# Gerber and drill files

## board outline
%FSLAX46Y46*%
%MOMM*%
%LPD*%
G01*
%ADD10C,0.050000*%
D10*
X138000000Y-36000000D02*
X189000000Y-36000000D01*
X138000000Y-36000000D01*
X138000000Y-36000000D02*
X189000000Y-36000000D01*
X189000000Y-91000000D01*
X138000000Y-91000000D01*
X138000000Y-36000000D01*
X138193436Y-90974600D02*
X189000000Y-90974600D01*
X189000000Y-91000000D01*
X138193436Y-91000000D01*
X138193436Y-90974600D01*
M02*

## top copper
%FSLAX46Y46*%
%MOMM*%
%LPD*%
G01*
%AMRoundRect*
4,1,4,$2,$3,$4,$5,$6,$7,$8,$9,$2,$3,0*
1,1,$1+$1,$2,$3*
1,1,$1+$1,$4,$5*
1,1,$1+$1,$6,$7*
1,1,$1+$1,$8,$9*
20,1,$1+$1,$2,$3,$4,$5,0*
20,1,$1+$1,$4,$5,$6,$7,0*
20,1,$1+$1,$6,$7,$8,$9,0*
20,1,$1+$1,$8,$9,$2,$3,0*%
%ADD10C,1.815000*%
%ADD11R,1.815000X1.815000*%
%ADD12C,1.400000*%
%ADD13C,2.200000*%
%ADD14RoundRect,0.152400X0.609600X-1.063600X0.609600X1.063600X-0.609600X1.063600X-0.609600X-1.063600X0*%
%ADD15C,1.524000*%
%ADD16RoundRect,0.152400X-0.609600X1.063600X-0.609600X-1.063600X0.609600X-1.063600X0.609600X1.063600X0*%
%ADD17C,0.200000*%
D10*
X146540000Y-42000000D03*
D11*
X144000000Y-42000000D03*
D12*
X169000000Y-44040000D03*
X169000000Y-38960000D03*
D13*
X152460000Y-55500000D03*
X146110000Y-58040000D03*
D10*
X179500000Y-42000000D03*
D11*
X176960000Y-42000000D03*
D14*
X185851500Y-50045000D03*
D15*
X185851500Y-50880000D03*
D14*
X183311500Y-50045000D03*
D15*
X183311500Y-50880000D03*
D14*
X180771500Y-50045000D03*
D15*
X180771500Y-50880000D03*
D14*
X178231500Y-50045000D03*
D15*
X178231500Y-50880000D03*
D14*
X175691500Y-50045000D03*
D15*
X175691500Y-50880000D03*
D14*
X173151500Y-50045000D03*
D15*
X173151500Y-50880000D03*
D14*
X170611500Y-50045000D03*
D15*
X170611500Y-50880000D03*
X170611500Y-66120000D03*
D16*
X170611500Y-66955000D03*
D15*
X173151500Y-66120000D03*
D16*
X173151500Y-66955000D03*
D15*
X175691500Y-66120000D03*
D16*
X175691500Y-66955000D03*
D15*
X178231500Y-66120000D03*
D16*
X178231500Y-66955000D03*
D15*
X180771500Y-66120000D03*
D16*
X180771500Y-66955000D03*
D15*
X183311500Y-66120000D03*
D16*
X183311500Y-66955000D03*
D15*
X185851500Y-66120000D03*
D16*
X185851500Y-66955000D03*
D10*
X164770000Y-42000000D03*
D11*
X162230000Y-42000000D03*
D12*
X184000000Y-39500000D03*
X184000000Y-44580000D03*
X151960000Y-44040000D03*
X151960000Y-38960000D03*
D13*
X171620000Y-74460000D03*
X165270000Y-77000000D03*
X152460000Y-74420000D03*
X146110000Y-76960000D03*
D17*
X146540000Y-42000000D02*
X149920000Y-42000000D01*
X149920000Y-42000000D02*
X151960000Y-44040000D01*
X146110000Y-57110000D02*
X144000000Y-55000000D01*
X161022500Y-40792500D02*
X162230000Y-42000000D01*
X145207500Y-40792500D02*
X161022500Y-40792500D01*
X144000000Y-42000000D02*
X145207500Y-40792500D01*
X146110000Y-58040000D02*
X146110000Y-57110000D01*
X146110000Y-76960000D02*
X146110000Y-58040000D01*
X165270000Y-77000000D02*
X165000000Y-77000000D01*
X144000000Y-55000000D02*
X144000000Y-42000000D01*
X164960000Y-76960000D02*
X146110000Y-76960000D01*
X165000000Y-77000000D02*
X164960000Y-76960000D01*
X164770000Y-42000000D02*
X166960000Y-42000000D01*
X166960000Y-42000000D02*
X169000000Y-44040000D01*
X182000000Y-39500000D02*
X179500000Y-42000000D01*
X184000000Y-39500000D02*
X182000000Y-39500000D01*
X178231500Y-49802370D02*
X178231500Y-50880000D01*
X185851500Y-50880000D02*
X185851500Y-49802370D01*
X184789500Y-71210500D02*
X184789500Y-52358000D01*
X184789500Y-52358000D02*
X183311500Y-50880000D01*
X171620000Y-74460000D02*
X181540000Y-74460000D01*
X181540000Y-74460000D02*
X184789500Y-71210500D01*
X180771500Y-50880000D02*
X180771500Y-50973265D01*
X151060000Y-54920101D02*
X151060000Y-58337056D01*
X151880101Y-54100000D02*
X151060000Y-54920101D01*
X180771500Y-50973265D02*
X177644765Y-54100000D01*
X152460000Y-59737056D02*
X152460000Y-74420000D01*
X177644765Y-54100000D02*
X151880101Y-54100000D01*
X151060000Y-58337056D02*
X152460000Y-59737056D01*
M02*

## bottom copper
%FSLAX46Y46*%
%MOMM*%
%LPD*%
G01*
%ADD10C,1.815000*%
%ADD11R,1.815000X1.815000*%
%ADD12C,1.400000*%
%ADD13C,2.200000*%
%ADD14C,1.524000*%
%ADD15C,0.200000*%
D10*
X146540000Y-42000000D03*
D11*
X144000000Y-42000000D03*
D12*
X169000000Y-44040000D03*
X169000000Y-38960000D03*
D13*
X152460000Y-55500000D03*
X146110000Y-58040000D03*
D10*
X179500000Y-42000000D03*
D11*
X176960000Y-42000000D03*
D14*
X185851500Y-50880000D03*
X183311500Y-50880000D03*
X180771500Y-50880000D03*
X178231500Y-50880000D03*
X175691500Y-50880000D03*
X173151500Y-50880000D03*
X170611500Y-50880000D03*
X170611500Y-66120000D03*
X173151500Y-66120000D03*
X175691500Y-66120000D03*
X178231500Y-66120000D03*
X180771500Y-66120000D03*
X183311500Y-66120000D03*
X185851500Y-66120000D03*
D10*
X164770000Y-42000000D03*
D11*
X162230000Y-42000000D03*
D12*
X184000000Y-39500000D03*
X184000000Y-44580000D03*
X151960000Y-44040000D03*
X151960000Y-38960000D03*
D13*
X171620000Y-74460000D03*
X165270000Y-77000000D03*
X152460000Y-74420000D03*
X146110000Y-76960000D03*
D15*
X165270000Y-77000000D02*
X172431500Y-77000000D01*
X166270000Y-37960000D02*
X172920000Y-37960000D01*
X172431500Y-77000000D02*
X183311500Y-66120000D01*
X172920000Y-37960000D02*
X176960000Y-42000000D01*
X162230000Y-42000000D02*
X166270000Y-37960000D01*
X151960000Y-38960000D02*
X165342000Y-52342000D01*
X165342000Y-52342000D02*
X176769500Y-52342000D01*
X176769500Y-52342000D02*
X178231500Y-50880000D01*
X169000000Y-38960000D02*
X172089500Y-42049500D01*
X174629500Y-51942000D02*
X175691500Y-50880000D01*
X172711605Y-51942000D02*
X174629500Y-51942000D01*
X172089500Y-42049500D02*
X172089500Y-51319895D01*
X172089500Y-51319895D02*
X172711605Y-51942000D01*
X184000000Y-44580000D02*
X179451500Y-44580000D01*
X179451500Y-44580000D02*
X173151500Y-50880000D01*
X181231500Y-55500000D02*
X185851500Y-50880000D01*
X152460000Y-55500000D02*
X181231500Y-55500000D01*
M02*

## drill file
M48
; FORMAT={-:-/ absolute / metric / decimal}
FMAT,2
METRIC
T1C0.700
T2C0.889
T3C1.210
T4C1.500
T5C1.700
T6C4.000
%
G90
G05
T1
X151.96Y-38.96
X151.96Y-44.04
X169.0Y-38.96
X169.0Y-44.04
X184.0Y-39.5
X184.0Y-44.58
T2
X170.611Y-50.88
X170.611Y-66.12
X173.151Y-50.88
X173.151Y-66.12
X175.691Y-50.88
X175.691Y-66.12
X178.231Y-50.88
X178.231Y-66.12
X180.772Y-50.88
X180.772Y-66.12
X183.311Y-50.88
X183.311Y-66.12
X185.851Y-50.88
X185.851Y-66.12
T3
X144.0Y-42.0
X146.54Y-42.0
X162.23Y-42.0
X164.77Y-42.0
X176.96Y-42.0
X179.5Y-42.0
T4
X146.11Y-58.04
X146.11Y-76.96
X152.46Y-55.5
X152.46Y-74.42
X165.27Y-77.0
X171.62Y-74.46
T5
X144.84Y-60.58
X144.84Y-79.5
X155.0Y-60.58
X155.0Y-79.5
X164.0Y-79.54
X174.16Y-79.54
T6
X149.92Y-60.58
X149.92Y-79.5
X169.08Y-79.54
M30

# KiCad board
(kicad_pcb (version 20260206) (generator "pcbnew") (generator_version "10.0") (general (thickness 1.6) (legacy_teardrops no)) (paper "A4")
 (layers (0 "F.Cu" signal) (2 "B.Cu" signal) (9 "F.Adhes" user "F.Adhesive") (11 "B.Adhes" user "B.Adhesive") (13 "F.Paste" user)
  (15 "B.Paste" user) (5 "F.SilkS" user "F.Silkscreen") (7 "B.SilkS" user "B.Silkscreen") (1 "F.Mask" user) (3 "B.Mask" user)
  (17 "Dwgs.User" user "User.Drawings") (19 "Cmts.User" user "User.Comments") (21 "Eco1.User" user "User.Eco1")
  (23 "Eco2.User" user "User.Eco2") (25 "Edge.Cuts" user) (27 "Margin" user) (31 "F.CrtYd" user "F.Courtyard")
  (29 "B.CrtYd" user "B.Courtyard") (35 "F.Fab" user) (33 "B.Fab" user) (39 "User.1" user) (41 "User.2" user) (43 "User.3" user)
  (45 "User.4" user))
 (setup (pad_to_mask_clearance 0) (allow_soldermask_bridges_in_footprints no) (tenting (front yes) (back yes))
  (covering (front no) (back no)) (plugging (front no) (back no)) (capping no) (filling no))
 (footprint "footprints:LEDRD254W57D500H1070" (layer "F.Cu") (at 145.27 42)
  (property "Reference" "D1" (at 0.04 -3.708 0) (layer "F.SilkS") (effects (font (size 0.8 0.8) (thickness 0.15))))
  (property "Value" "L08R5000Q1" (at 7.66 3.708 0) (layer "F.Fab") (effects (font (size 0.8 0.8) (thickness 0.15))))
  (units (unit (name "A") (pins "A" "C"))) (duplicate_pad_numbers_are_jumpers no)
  (pad "A" thru_hole circle (at 1.27 0) (size 1.815 1.815) (drill 1.21) (layers "*.Cu" "*.Mask") (remove_unused_layers no)
   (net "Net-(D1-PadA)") (solder_mask_margin 0.102))
  (pad "C" thru_hole rect (at -1.27 0) (size 1.815 1.815) (drill 1.21) (layers "*.Cu" "*.Mask") (remove_unused_layers no) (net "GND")
   (solder_mask_margin 0.102)))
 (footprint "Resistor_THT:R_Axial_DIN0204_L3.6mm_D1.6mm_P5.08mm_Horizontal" (layer "F.Cu") (at 169 44.04 90)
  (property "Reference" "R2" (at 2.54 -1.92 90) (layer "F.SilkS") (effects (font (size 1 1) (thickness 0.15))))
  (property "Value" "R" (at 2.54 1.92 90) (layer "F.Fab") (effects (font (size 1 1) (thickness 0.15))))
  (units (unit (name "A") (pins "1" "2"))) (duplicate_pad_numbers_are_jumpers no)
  (pad "1" thru_hole circle (at 0 0 90) (size 1.4 1.4) (drill 0.7) (layers "*.Cu" "*.Mask") (remove_unused_layers no) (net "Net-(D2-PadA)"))
  (pad "2" thru_hole circle (at 5.08 0 90) (size 1.4 1.4) (drill 0.7) (layers "*.Cu" "*.Mask") (remove_unused_layers no) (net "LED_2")))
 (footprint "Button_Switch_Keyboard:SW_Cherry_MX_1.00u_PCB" (layer "F.Cu") (at 152.46 55.5)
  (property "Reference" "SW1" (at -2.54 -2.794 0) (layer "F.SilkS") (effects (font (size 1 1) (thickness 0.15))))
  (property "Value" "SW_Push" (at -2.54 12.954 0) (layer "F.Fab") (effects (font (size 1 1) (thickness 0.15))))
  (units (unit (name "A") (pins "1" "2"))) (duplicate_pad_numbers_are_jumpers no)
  (pad "" np_thru_hole circle (at -7.62 5.08) (size 1.7 1.7) (drill 1.7) (layers "*.Cu" "*.Mask"))
  (pad "" np_thru_hole circle (at -2.54 5.08) (size 4 4) (drill 4) (layers "*.Cu" "*.Mask"))
  (pad "" np_thru_hole circle (at 2.54 5.08) (size 1.7 1.7) (drill 1.7) (layers "*.Cu" "*.Mask"))
  (pad "1" thru_hole circle (at 0 0) (size 2.2 2.2) (drill 1.5) (layers "*.Cu" "*.Mask") (remove_unused_layers no) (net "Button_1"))
  (pad "2" thru_hole circle (at -6.35 2.54) (size 2.2 2.2) (drill 1.5) (layers "*.Cu" "*.Mask") (remove_unused_layers no) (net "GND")))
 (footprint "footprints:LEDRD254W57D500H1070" (layer "F.Cu") (at 178.23 42)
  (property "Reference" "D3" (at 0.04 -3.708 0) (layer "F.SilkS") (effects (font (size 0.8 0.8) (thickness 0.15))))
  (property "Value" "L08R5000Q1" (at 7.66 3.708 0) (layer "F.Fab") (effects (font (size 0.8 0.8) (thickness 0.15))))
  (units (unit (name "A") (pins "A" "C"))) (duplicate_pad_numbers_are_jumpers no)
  (pad "A" thru_hole circle (at 1.27 0) (size 1.815 1.815) (drill 1.21) (layers "*.Cu" "*.Mask") (remove_unused_layers no)
   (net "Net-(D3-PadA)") (solder_mask_margin 0.102))
  (pad "C" thru_hole rect (at -1.27 0) (size 1.815 1.815) (drill 1.21) (layers "*.Cu" "*.Mask") (remove_unused_layers no) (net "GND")
   (solder_mask_margin 0.102)))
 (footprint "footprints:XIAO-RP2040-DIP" (layer "F.Cu") (at 178.2315 58.5)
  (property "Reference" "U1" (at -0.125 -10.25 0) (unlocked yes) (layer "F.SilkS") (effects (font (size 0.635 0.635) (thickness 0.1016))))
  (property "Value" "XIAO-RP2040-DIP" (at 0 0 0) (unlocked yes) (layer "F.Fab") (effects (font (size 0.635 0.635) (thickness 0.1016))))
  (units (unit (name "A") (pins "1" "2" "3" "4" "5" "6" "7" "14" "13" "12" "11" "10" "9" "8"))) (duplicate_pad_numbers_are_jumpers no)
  (pad "1" smd roundrect (at 7.62 -8.455 90) (size 2.432 1.524) (layers "F.Cu" "F.Mask") (roundrect_rratio 0.1) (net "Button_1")
   (thermal_bridge_angle 45))
  (pad "1" thru_hole circle (at 7.62 -7.62 90) (size 1.524 1.524) (drill 0.889) (layers "*.Cu" "*.Mask") (remove_unused_layers no)
   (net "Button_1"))
  (pad "2" smd roundrect (at 5.08 -8.455 90) (size 2.432 1.524) (layers "F.Cu" "F.Mask") (roundrect_rratio 0.1) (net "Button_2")
   (thermal_bridge_angle 45))
  (pad "2" thru_hole circle (at 5.08 -7.62 90) (size 1.524 1.524) (drill 0.889) (layers "*.Cu" "*.Mask") (remove_unused_layers no)
   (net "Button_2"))
  (pad "3" smd roundrect (at 2.54 -8.455 90) (size 2.432 1.524) (layers "F.Cu" "F.Mask") (roundrect_rratio 0.1) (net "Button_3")
   (thermal_bridge_angle 45))
  (pad "3" thru_hole circle (at 2.54 -7.62 90) (size 1.524 1.524) (drill 0.889) (layers "*.Cu" "*.Mask") (remove_unused_layers no)
   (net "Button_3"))
  (pad "4" smd roundrect (at 0 -8.455 90) (size 2.432 1.524) (layers "F.Cu" "F.Mask") (roundrect_rratio 0.1) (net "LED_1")
   (thermal_bridge_angle 45))
  (pad "4" thru_hole circle (at 0 -7.62 90) (size 1.524 1.524) (drill 0.889) (layers "*.Cu" "*.Mask") (remove_unused_layers no)
   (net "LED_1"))
  (pad "5" smd roundrect (at -2.54 -8.455 90) (size 2.432 1.524) (layers "F.Cu" "F.Mask") (roundrect_rratio 0.1) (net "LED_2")
   (thermal_bridge_angle 45))
  (pad "5" thru_hole circle (at -2.54 -7.62 90) (size 1.524 1.524) (drill 0.889) (layers "*.Cu" "*.Mask") (remove_unused_layers no)
   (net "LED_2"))
  (pad "6" smd roundrect (at -5.08 -8.455 90) (size 2.432 1.524) (layers "F.Cu" "F.Mask") (roundrect_rratio 0.1) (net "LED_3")
   (thermal_bridge_angle 45))
  (pad "6" thru_hole circle (at -5.08 -7.62 90) (size 1.524 1.524) (drill 0.889) (layers "*.Cu" "*.Mask") (remove_unused_layers no)
   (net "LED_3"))
  (pad "7" smd roundrect (at -7.62 -8.455 90) (size 2.432 1.524) (layers "F.Cu" "F.Mask") (roundrect_rratio 0.1)
   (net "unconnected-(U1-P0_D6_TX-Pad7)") (thermal_bridge_angle 45))
  (pad "7" thru_hole circle (at -7.62 -7.62 90) (size 1.524 1.524) (drill 0.889) (layers "*.Cu" "*.Mask") (remove_unused_layers no)
   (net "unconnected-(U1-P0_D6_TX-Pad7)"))
  (pad "8" thru_hole circle (at -7.62 7.62 270) (size 1.524 1.524) (drill 0.889) (layers "*.Cu" "*.Mask") (remove_unused_layers no)
   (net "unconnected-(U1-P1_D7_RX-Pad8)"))
  (pad "8" smd roundrect (at -7.62 8.455 270) (size 2.432 1.524) (layers "F.Cu" "F.Mask") (roundrect_rratio 0.1)
   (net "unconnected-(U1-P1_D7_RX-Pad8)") (thermal_bridge_angle 45))
  (pad "9" thru_hole circle (at -5.08 7.62 270) (size 1.524 1.524) (drill 0.889) (layers "*.Cu" "*.Mask") (remove_unused_layers no)
   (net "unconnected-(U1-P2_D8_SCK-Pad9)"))
  (pad "9" smd roundrect (at -5.08 8.455 270) (size 2.432 1.524) (layers "F.Cu" "F.Mask") (roundrect_rratio 0.1)
   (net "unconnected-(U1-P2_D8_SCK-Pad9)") (thermal_bridge_angle 45))
  (pad "10" thru_hole circle (at -2.54 7.62 270) (size 1.524 1.524) (drill 0.889) (layers "*.Cu" "*.Mask") (remove_unused_layers no)
   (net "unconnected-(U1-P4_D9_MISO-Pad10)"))
  (pad "10" smd roundrect (at -2.54 8.455 270) (size 2.432 1.524) (layers "F.Cu" "F.Mask") (roundrect_rratio 0.1)
   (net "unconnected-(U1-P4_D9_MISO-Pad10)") (thermal_bridge_angle 45))
  (pad "11" thru_hole circle (at 0 7.62 270) (size 1.524 1.524) (drill 0.889) (layers "*.Cu" "*.Mask") (remove_unused_layers no)
   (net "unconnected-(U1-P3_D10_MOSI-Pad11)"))
  (pad "11" smd roundrect (at 0 8.455 270) (size 2.432 1.524) (layers "F.Cu" "F.Mask") (roundrect_rratio 0.1)
   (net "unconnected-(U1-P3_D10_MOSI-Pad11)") (thermal_bridge_angle 45))
  (pad "12" thru_hole circle (at 2.54 7.62 270) (size 1.524 1.524) (drill 0.889) (layers "*.Cu" "*.Mask") (remove_unused_layers no)
   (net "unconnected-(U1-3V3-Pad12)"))
  (pad "12" smd roundrect (at 2.54 8.455 270) (size 2.432 1.524) (layers "F.Cu" "F.Mask") (roundrect_rratio 0.1)
   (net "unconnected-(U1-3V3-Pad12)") (thermal_bridge_angle 45))
  (pad "13" thru_hole circle (at 5.08 7.62 270) (size 1.524 1.524) (drill 0.889) (layers "*.Cu" "*.Mask") (remove_unused_layers no)
   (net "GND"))
  (pad "13" smd roundrect (at 5.08 8.455 270) (size 2.432 1.524) (layers "F.Cu" "F.Mask") (roundrect_rratio 0.1) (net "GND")
   (thermal_bridge_angle 45))
  (pad "14" thru_hole circle (at 7.62 7.62 270) (size 1.524 1.524) (drill 0.889) (layers "*.Cu" "*.Mask") (remove_unused_layers no)
   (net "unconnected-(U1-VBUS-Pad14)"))
  (pad "14" smd roundrect (at 7.62 8.455 270) (size 2.432 1.524) (layers "F.Cu" "F.Mask") (roundrect_rratio 0.1)
   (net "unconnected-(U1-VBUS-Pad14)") (thermal_bridge_angle 45)))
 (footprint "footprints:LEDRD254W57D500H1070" (layer "F.Cu") (at 163.5 42)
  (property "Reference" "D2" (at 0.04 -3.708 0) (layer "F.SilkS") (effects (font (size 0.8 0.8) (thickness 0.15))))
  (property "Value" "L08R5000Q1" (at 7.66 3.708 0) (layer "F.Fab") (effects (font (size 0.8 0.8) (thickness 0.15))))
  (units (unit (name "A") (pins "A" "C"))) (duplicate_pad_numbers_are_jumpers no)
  (pad "A" thru_hole circle (at 1.27 0) (size 1.815 1.815) (drill 1.21) (layers "*.Cu" "*.Mask") (remove_unused_layers no)
   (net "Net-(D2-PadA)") (solder_mask_margin 0.102))
  (pad "C" thru_hole rect (at -1.27 0) (size 1.815 1.815) (drill 1.21) (layers "*.Cu" "*.Mask") (remove_unused_layers no) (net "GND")
   (solder_mask_margin 0.102)))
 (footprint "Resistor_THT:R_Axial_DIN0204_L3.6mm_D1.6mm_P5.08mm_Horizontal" (layer "F.Cu") (at 184 39.5 -90)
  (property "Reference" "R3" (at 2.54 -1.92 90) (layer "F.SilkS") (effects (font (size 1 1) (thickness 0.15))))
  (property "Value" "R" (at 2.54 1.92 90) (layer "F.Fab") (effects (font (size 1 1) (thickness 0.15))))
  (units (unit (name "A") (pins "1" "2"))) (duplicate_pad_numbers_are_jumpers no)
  (pad "1" thru_hole circle (at 0 0 270) (size 1.4 1.4) (drill 0.7) (layers "*.Cu" "*.Mask") (remove_unused_layers no) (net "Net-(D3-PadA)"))
  (pad "2" thru_hole circle (at 5.08 0 270) (size 1.4 1.4) (drill 0.7) (layers "*.Cu" "*.Mask") (remove_unused_layers no) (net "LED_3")))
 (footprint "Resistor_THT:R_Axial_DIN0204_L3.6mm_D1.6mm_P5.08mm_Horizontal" (layer "F.Cu") (at 151.96 44.04 90)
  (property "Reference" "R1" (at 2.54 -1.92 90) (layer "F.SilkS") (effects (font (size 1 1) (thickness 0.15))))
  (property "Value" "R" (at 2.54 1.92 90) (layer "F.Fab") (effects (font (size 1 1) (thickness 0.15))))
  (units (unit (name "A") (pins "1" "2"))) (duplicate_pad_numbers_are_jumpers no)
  (pad "1" thru_hole circle (at 0 0 90) (size 1.4 1.4) (drill 0.7) (layers "*.Cu" "*.Mask") (remove_unused_layers no) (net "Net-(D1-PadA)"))
  (pad "2" thru_hole circle (at 5.08 0 90) (size 1.4 1.4) (drill 0.7) (layers "*.Cu" "*.Mask") (remove_unused_layers no) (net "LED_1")))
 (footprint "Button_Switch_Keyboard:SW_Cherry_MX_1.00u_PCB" (layer "F.Cu") (at 171.62 74.46)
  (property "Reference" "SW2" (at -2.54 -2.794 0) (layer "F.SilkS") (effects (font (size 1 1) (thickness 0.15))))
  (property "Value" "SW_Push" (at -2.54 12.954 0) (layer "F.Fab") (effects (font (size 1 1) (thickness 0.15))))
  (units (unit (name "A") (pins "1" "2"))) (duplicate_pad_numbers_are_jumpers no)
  (pad "" np_thru_hole circle (at -7.62 5.08) (size 1.7 1.7) (drill 1.7) (layers "*.Cu" "*.Mask"))
  (pad "" np_thru_hole circle (at -2.54 5.08) (size 4 4) (drill 4) (layers "*.Cu" "*.Mask"))
  (pad "" np_thru_hole circle (at 2.54 5.08) (size 1.7 1.7) (drill 1.7) (layers "*.Cu" "*.Mask"))
  (pad "1" thru_hole circle (at 0 0) (size 2.2 2.2) (drill 1.5) (layers "*.Cu" "*.Mask") (remove_unused_layers no) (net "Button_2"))
  (pad "2" thru_hole circle (at -6.35 2.54) (size 2.2 2.2) (drill 1.5) (layers "*.Cu" "*.Mask") (remove_unused_layers no) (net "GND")))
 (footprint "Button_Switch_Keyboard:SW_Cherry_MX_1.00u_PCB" (layer "F.Cu") (at 152.46 74.42)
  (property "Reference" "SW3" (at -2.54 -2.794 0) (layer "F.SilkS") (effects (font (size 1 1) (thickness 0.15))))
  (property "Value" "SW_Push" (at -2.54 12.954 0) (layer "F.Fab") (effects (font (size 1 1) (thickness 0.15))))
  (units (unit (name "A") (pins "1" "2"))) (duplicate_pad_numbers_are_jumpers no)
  (pad "" np_thru_hole circle (at -7.62 5.08) (size 1.7 1.7) (drill 1.7) (layers "*.Cu" "*.Mask"))
  (pad "" np_thru_hole circle (at -2.54 5.08) (size 4 4) (drill 4) (layers "*.Cu" "*.Mask"))
  (pad "" np_thru_hole circle (at 2.54 5.08) (size 1.7 1.7) (drill 1.7) (layers "*.Cu" "*.Mask"))
  (pad "1" thru_hole circle (at 0 0) (size 2.2 2.2) (drill 1.5) (layers "*.Cu" "*.Mask") (remove_unused_layers no) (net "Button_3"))
  (pad "2" thru_hole circle (at -6.35 2.54) (size 2.2 2.2) (drill 1.5) (layers "*.Cu" "*.Mask") (remove_unused_layers no) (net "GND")))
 (gr_rect (start 138 36) (end 189 36) (stroke (width 0.05) (type default)) (fill no) (layer "Edge.Cuts"))
 (gr_rect (start 138 36) (end 189 91) (stroke (width 0.05) (type default)) (fill no) (layer "Edge.Cuts"))
 (gr_rect (start 138.193436 90.9746) (end 189 91) (stroke (width 0.05) (type default)) (fill no) (layer "Edge.Cuts"))
 (segment (start 146.54 42) (end 149.92 42) (width 0.2) (layer "F.Cu") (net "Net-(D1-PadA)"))
 (segment (start 149.92 42) (end 151.96 44.04) (width 0.2) (layer "F.Cu") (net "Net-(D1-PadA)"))
 (segment (start 146.11 57.11) (end 144 55) (width 0.2) (layer "F.Cu") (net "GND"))
 (segment (start 161.0225 40.7925) (end 162.23 42) (width 0.2) (layer "F.Cu") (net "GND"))
 (segment (start 145.2075 40.7925) (end 161.0225 40.7925) (width 0.2) (layer "F.Cu") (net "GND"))
 (segment (start 144 42) (end 145.2075 40.7925) (width 0.2) (layer "F.Cu") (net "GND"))
 (segment (start 146.11 58.04) (end 146.11 57.11) (width 0.2) (layer "F.Cu") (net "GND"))
 (segment (start 146.11 76.96) (end 146.11 58.04) (width 0.2) (layer "F.Cu") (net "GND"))
 (segment (start 165.27 77) (end 165 77) (width 0.2) (layer "F.Cu") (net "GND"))
 (segment (start 144 55) (end 144 42) (width 0.2) (layer "F.Cu") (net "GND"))
 (segment (start 164.96 76.96) (end 146.11 76.96) (width 0.2) (layer "F.Cu") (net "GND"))
 (segment (start 165 77) (end 164.96 76.96) (width 0.2) (layer "F.Cu") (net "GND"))
 (segment (start 165.27 77) (end 172.4315 77) (width 0.2) (layer "B.Cu") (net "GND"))
 (segment (start 166.27 37.96) (end 172.92 37.96) (width 0.2) (layer "B.Cu") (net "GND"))
 (segment (start 172.4315 77) (end 183.3115 66.12) (width 0.2) (layer "B.Cu") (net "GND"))
 (segment (start 172.92 37.96) (end 176.96 42) (width 0.2) (layer "B.Cu") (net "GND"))
 (segment (start 162.23 42) (end 166.27 37.96) (width 0.2) (layer "B.Cu") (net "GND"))
 (segment (start 164.77 42) (end 166.96 42) (width 0.2) (layer "F.Cu") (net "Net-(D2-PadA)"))
 (segment (start 166.96 42) (end 169 44.04) (width 0.2) (layer "F.Cu") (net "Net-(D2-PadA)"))
 (segment (start 182 39.5) (end 179.5 42) (width 0.2) (layer "F.Cu") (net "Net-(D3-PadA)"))
 (segment (start 184 39.5) (end 182 39.5) (width 0.2) (layer "F.Cu") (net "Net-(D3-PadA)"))
 (segment (start 178.2315 49.80237) (end 178.2315 50.88) (width 0.2) (layer "F.Cu") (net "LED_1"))
 (segment (start 151.96 38.96) (end 165.342 52.342) (width 0.2) (layer "B.Cu") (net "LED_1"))
 (segment (start 165.342 52.342) (end 176.7695 52.342) (width 0.2) (layer "B.Cu") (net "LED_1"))
 (segment (start 176.7695 52.342) (end 178.2315 50.88) (width 0.2) (layer "B.Cu") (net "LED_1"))
 (segment (start 169 38.96) (end 172.0895 42.0495) (width 0.2) (layer "B.Cu") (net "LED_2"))
 (segment (start 174.6295 51.942) (end 175.6915 50.88) (width 0.2) (layer "B.Cu") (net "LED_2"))
 (segment (start 172.711605 51.942) (end 174.6295 51.942) (width 0.2) (layer "B.Cu") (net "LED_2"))
 (segment (start 172.0895 42.0495) (end 172.0895 51.319895) (width 0.2) (layer "B.Cu") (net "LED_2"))
 (segment (start 172.0895 51.319895) (end 172.711605 51.942) (width 0.2) (layer "B.Cu") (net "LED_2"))
 (segment (start 184 44.58) (end 179.4515 44.58) (width 0.2) (layer "B.Cu") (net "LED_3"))
 (segment (start 179.4515 44.58) (end 173.1515 50.88) (width 0.2) (layer "B.Cu") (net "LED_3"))
 (segment (start 185.8515 50.88) (end 185.8515 49.80237) (width 0.2) (layer "F.Cu") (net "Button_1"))
 (segment (start 181.2315 55.5) (end 185.8515 50.88) (width 0.2) (layer "B.Cu") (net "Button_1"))
 (segment (start 152.46 55.5) (end 181.2315 55.5) (width 0.2) (layer "B.Cu") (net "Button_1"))
 (segment (start 184.7895 71.2105) (end 184.7895 52.358) (width 0.2) (layer "F.Cu") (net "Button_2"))
 (segment (start 184.7895 52.358) (end 183.3115 50.88) (width 0.2) (layer "F.Cu") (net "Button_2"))
 (segment (start 171.62 74.46) (end 181.54 74.46) (width 0.2) (layer "F.Cu") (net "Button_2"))
 (segment (start 181.54 74.46) (end 184.7895 71.2105) (width 0.2) (layer "F.Cu") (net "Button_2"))
 (segment (start 180.7715 50.88) (end 180.7715 50.973265) (width 0.2) (layer "F.Cu") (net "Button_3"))
 (segment (start 151.06 54.920101) (end 151.06 58.337056) (width 0.2) (layer "F.Cu") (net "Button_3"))
 (segment (start 151.880101 54.1) (end 151.06 54.920101) (width 0.2) (layer "F.Cu") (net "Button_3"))
 (segment (start 180.7715 50.973265) (end 177.644765 54.1) (width 0.2) (layer "F.Cu") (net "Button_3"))
 (segment (start 152.46 59.737056) (end 152.46 74.42) (width 0.2) (layer "F.Cu") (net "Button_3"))
 (segment (start 177.644765 54.1) (end 151.880101 54.1) (width 0.2) (layer "F.Cu") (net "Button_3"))
 (segment (start 151.06 58.337056) (end 152.46 59.737056) (width 0.2) (layer "F.Cu") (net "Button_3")))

